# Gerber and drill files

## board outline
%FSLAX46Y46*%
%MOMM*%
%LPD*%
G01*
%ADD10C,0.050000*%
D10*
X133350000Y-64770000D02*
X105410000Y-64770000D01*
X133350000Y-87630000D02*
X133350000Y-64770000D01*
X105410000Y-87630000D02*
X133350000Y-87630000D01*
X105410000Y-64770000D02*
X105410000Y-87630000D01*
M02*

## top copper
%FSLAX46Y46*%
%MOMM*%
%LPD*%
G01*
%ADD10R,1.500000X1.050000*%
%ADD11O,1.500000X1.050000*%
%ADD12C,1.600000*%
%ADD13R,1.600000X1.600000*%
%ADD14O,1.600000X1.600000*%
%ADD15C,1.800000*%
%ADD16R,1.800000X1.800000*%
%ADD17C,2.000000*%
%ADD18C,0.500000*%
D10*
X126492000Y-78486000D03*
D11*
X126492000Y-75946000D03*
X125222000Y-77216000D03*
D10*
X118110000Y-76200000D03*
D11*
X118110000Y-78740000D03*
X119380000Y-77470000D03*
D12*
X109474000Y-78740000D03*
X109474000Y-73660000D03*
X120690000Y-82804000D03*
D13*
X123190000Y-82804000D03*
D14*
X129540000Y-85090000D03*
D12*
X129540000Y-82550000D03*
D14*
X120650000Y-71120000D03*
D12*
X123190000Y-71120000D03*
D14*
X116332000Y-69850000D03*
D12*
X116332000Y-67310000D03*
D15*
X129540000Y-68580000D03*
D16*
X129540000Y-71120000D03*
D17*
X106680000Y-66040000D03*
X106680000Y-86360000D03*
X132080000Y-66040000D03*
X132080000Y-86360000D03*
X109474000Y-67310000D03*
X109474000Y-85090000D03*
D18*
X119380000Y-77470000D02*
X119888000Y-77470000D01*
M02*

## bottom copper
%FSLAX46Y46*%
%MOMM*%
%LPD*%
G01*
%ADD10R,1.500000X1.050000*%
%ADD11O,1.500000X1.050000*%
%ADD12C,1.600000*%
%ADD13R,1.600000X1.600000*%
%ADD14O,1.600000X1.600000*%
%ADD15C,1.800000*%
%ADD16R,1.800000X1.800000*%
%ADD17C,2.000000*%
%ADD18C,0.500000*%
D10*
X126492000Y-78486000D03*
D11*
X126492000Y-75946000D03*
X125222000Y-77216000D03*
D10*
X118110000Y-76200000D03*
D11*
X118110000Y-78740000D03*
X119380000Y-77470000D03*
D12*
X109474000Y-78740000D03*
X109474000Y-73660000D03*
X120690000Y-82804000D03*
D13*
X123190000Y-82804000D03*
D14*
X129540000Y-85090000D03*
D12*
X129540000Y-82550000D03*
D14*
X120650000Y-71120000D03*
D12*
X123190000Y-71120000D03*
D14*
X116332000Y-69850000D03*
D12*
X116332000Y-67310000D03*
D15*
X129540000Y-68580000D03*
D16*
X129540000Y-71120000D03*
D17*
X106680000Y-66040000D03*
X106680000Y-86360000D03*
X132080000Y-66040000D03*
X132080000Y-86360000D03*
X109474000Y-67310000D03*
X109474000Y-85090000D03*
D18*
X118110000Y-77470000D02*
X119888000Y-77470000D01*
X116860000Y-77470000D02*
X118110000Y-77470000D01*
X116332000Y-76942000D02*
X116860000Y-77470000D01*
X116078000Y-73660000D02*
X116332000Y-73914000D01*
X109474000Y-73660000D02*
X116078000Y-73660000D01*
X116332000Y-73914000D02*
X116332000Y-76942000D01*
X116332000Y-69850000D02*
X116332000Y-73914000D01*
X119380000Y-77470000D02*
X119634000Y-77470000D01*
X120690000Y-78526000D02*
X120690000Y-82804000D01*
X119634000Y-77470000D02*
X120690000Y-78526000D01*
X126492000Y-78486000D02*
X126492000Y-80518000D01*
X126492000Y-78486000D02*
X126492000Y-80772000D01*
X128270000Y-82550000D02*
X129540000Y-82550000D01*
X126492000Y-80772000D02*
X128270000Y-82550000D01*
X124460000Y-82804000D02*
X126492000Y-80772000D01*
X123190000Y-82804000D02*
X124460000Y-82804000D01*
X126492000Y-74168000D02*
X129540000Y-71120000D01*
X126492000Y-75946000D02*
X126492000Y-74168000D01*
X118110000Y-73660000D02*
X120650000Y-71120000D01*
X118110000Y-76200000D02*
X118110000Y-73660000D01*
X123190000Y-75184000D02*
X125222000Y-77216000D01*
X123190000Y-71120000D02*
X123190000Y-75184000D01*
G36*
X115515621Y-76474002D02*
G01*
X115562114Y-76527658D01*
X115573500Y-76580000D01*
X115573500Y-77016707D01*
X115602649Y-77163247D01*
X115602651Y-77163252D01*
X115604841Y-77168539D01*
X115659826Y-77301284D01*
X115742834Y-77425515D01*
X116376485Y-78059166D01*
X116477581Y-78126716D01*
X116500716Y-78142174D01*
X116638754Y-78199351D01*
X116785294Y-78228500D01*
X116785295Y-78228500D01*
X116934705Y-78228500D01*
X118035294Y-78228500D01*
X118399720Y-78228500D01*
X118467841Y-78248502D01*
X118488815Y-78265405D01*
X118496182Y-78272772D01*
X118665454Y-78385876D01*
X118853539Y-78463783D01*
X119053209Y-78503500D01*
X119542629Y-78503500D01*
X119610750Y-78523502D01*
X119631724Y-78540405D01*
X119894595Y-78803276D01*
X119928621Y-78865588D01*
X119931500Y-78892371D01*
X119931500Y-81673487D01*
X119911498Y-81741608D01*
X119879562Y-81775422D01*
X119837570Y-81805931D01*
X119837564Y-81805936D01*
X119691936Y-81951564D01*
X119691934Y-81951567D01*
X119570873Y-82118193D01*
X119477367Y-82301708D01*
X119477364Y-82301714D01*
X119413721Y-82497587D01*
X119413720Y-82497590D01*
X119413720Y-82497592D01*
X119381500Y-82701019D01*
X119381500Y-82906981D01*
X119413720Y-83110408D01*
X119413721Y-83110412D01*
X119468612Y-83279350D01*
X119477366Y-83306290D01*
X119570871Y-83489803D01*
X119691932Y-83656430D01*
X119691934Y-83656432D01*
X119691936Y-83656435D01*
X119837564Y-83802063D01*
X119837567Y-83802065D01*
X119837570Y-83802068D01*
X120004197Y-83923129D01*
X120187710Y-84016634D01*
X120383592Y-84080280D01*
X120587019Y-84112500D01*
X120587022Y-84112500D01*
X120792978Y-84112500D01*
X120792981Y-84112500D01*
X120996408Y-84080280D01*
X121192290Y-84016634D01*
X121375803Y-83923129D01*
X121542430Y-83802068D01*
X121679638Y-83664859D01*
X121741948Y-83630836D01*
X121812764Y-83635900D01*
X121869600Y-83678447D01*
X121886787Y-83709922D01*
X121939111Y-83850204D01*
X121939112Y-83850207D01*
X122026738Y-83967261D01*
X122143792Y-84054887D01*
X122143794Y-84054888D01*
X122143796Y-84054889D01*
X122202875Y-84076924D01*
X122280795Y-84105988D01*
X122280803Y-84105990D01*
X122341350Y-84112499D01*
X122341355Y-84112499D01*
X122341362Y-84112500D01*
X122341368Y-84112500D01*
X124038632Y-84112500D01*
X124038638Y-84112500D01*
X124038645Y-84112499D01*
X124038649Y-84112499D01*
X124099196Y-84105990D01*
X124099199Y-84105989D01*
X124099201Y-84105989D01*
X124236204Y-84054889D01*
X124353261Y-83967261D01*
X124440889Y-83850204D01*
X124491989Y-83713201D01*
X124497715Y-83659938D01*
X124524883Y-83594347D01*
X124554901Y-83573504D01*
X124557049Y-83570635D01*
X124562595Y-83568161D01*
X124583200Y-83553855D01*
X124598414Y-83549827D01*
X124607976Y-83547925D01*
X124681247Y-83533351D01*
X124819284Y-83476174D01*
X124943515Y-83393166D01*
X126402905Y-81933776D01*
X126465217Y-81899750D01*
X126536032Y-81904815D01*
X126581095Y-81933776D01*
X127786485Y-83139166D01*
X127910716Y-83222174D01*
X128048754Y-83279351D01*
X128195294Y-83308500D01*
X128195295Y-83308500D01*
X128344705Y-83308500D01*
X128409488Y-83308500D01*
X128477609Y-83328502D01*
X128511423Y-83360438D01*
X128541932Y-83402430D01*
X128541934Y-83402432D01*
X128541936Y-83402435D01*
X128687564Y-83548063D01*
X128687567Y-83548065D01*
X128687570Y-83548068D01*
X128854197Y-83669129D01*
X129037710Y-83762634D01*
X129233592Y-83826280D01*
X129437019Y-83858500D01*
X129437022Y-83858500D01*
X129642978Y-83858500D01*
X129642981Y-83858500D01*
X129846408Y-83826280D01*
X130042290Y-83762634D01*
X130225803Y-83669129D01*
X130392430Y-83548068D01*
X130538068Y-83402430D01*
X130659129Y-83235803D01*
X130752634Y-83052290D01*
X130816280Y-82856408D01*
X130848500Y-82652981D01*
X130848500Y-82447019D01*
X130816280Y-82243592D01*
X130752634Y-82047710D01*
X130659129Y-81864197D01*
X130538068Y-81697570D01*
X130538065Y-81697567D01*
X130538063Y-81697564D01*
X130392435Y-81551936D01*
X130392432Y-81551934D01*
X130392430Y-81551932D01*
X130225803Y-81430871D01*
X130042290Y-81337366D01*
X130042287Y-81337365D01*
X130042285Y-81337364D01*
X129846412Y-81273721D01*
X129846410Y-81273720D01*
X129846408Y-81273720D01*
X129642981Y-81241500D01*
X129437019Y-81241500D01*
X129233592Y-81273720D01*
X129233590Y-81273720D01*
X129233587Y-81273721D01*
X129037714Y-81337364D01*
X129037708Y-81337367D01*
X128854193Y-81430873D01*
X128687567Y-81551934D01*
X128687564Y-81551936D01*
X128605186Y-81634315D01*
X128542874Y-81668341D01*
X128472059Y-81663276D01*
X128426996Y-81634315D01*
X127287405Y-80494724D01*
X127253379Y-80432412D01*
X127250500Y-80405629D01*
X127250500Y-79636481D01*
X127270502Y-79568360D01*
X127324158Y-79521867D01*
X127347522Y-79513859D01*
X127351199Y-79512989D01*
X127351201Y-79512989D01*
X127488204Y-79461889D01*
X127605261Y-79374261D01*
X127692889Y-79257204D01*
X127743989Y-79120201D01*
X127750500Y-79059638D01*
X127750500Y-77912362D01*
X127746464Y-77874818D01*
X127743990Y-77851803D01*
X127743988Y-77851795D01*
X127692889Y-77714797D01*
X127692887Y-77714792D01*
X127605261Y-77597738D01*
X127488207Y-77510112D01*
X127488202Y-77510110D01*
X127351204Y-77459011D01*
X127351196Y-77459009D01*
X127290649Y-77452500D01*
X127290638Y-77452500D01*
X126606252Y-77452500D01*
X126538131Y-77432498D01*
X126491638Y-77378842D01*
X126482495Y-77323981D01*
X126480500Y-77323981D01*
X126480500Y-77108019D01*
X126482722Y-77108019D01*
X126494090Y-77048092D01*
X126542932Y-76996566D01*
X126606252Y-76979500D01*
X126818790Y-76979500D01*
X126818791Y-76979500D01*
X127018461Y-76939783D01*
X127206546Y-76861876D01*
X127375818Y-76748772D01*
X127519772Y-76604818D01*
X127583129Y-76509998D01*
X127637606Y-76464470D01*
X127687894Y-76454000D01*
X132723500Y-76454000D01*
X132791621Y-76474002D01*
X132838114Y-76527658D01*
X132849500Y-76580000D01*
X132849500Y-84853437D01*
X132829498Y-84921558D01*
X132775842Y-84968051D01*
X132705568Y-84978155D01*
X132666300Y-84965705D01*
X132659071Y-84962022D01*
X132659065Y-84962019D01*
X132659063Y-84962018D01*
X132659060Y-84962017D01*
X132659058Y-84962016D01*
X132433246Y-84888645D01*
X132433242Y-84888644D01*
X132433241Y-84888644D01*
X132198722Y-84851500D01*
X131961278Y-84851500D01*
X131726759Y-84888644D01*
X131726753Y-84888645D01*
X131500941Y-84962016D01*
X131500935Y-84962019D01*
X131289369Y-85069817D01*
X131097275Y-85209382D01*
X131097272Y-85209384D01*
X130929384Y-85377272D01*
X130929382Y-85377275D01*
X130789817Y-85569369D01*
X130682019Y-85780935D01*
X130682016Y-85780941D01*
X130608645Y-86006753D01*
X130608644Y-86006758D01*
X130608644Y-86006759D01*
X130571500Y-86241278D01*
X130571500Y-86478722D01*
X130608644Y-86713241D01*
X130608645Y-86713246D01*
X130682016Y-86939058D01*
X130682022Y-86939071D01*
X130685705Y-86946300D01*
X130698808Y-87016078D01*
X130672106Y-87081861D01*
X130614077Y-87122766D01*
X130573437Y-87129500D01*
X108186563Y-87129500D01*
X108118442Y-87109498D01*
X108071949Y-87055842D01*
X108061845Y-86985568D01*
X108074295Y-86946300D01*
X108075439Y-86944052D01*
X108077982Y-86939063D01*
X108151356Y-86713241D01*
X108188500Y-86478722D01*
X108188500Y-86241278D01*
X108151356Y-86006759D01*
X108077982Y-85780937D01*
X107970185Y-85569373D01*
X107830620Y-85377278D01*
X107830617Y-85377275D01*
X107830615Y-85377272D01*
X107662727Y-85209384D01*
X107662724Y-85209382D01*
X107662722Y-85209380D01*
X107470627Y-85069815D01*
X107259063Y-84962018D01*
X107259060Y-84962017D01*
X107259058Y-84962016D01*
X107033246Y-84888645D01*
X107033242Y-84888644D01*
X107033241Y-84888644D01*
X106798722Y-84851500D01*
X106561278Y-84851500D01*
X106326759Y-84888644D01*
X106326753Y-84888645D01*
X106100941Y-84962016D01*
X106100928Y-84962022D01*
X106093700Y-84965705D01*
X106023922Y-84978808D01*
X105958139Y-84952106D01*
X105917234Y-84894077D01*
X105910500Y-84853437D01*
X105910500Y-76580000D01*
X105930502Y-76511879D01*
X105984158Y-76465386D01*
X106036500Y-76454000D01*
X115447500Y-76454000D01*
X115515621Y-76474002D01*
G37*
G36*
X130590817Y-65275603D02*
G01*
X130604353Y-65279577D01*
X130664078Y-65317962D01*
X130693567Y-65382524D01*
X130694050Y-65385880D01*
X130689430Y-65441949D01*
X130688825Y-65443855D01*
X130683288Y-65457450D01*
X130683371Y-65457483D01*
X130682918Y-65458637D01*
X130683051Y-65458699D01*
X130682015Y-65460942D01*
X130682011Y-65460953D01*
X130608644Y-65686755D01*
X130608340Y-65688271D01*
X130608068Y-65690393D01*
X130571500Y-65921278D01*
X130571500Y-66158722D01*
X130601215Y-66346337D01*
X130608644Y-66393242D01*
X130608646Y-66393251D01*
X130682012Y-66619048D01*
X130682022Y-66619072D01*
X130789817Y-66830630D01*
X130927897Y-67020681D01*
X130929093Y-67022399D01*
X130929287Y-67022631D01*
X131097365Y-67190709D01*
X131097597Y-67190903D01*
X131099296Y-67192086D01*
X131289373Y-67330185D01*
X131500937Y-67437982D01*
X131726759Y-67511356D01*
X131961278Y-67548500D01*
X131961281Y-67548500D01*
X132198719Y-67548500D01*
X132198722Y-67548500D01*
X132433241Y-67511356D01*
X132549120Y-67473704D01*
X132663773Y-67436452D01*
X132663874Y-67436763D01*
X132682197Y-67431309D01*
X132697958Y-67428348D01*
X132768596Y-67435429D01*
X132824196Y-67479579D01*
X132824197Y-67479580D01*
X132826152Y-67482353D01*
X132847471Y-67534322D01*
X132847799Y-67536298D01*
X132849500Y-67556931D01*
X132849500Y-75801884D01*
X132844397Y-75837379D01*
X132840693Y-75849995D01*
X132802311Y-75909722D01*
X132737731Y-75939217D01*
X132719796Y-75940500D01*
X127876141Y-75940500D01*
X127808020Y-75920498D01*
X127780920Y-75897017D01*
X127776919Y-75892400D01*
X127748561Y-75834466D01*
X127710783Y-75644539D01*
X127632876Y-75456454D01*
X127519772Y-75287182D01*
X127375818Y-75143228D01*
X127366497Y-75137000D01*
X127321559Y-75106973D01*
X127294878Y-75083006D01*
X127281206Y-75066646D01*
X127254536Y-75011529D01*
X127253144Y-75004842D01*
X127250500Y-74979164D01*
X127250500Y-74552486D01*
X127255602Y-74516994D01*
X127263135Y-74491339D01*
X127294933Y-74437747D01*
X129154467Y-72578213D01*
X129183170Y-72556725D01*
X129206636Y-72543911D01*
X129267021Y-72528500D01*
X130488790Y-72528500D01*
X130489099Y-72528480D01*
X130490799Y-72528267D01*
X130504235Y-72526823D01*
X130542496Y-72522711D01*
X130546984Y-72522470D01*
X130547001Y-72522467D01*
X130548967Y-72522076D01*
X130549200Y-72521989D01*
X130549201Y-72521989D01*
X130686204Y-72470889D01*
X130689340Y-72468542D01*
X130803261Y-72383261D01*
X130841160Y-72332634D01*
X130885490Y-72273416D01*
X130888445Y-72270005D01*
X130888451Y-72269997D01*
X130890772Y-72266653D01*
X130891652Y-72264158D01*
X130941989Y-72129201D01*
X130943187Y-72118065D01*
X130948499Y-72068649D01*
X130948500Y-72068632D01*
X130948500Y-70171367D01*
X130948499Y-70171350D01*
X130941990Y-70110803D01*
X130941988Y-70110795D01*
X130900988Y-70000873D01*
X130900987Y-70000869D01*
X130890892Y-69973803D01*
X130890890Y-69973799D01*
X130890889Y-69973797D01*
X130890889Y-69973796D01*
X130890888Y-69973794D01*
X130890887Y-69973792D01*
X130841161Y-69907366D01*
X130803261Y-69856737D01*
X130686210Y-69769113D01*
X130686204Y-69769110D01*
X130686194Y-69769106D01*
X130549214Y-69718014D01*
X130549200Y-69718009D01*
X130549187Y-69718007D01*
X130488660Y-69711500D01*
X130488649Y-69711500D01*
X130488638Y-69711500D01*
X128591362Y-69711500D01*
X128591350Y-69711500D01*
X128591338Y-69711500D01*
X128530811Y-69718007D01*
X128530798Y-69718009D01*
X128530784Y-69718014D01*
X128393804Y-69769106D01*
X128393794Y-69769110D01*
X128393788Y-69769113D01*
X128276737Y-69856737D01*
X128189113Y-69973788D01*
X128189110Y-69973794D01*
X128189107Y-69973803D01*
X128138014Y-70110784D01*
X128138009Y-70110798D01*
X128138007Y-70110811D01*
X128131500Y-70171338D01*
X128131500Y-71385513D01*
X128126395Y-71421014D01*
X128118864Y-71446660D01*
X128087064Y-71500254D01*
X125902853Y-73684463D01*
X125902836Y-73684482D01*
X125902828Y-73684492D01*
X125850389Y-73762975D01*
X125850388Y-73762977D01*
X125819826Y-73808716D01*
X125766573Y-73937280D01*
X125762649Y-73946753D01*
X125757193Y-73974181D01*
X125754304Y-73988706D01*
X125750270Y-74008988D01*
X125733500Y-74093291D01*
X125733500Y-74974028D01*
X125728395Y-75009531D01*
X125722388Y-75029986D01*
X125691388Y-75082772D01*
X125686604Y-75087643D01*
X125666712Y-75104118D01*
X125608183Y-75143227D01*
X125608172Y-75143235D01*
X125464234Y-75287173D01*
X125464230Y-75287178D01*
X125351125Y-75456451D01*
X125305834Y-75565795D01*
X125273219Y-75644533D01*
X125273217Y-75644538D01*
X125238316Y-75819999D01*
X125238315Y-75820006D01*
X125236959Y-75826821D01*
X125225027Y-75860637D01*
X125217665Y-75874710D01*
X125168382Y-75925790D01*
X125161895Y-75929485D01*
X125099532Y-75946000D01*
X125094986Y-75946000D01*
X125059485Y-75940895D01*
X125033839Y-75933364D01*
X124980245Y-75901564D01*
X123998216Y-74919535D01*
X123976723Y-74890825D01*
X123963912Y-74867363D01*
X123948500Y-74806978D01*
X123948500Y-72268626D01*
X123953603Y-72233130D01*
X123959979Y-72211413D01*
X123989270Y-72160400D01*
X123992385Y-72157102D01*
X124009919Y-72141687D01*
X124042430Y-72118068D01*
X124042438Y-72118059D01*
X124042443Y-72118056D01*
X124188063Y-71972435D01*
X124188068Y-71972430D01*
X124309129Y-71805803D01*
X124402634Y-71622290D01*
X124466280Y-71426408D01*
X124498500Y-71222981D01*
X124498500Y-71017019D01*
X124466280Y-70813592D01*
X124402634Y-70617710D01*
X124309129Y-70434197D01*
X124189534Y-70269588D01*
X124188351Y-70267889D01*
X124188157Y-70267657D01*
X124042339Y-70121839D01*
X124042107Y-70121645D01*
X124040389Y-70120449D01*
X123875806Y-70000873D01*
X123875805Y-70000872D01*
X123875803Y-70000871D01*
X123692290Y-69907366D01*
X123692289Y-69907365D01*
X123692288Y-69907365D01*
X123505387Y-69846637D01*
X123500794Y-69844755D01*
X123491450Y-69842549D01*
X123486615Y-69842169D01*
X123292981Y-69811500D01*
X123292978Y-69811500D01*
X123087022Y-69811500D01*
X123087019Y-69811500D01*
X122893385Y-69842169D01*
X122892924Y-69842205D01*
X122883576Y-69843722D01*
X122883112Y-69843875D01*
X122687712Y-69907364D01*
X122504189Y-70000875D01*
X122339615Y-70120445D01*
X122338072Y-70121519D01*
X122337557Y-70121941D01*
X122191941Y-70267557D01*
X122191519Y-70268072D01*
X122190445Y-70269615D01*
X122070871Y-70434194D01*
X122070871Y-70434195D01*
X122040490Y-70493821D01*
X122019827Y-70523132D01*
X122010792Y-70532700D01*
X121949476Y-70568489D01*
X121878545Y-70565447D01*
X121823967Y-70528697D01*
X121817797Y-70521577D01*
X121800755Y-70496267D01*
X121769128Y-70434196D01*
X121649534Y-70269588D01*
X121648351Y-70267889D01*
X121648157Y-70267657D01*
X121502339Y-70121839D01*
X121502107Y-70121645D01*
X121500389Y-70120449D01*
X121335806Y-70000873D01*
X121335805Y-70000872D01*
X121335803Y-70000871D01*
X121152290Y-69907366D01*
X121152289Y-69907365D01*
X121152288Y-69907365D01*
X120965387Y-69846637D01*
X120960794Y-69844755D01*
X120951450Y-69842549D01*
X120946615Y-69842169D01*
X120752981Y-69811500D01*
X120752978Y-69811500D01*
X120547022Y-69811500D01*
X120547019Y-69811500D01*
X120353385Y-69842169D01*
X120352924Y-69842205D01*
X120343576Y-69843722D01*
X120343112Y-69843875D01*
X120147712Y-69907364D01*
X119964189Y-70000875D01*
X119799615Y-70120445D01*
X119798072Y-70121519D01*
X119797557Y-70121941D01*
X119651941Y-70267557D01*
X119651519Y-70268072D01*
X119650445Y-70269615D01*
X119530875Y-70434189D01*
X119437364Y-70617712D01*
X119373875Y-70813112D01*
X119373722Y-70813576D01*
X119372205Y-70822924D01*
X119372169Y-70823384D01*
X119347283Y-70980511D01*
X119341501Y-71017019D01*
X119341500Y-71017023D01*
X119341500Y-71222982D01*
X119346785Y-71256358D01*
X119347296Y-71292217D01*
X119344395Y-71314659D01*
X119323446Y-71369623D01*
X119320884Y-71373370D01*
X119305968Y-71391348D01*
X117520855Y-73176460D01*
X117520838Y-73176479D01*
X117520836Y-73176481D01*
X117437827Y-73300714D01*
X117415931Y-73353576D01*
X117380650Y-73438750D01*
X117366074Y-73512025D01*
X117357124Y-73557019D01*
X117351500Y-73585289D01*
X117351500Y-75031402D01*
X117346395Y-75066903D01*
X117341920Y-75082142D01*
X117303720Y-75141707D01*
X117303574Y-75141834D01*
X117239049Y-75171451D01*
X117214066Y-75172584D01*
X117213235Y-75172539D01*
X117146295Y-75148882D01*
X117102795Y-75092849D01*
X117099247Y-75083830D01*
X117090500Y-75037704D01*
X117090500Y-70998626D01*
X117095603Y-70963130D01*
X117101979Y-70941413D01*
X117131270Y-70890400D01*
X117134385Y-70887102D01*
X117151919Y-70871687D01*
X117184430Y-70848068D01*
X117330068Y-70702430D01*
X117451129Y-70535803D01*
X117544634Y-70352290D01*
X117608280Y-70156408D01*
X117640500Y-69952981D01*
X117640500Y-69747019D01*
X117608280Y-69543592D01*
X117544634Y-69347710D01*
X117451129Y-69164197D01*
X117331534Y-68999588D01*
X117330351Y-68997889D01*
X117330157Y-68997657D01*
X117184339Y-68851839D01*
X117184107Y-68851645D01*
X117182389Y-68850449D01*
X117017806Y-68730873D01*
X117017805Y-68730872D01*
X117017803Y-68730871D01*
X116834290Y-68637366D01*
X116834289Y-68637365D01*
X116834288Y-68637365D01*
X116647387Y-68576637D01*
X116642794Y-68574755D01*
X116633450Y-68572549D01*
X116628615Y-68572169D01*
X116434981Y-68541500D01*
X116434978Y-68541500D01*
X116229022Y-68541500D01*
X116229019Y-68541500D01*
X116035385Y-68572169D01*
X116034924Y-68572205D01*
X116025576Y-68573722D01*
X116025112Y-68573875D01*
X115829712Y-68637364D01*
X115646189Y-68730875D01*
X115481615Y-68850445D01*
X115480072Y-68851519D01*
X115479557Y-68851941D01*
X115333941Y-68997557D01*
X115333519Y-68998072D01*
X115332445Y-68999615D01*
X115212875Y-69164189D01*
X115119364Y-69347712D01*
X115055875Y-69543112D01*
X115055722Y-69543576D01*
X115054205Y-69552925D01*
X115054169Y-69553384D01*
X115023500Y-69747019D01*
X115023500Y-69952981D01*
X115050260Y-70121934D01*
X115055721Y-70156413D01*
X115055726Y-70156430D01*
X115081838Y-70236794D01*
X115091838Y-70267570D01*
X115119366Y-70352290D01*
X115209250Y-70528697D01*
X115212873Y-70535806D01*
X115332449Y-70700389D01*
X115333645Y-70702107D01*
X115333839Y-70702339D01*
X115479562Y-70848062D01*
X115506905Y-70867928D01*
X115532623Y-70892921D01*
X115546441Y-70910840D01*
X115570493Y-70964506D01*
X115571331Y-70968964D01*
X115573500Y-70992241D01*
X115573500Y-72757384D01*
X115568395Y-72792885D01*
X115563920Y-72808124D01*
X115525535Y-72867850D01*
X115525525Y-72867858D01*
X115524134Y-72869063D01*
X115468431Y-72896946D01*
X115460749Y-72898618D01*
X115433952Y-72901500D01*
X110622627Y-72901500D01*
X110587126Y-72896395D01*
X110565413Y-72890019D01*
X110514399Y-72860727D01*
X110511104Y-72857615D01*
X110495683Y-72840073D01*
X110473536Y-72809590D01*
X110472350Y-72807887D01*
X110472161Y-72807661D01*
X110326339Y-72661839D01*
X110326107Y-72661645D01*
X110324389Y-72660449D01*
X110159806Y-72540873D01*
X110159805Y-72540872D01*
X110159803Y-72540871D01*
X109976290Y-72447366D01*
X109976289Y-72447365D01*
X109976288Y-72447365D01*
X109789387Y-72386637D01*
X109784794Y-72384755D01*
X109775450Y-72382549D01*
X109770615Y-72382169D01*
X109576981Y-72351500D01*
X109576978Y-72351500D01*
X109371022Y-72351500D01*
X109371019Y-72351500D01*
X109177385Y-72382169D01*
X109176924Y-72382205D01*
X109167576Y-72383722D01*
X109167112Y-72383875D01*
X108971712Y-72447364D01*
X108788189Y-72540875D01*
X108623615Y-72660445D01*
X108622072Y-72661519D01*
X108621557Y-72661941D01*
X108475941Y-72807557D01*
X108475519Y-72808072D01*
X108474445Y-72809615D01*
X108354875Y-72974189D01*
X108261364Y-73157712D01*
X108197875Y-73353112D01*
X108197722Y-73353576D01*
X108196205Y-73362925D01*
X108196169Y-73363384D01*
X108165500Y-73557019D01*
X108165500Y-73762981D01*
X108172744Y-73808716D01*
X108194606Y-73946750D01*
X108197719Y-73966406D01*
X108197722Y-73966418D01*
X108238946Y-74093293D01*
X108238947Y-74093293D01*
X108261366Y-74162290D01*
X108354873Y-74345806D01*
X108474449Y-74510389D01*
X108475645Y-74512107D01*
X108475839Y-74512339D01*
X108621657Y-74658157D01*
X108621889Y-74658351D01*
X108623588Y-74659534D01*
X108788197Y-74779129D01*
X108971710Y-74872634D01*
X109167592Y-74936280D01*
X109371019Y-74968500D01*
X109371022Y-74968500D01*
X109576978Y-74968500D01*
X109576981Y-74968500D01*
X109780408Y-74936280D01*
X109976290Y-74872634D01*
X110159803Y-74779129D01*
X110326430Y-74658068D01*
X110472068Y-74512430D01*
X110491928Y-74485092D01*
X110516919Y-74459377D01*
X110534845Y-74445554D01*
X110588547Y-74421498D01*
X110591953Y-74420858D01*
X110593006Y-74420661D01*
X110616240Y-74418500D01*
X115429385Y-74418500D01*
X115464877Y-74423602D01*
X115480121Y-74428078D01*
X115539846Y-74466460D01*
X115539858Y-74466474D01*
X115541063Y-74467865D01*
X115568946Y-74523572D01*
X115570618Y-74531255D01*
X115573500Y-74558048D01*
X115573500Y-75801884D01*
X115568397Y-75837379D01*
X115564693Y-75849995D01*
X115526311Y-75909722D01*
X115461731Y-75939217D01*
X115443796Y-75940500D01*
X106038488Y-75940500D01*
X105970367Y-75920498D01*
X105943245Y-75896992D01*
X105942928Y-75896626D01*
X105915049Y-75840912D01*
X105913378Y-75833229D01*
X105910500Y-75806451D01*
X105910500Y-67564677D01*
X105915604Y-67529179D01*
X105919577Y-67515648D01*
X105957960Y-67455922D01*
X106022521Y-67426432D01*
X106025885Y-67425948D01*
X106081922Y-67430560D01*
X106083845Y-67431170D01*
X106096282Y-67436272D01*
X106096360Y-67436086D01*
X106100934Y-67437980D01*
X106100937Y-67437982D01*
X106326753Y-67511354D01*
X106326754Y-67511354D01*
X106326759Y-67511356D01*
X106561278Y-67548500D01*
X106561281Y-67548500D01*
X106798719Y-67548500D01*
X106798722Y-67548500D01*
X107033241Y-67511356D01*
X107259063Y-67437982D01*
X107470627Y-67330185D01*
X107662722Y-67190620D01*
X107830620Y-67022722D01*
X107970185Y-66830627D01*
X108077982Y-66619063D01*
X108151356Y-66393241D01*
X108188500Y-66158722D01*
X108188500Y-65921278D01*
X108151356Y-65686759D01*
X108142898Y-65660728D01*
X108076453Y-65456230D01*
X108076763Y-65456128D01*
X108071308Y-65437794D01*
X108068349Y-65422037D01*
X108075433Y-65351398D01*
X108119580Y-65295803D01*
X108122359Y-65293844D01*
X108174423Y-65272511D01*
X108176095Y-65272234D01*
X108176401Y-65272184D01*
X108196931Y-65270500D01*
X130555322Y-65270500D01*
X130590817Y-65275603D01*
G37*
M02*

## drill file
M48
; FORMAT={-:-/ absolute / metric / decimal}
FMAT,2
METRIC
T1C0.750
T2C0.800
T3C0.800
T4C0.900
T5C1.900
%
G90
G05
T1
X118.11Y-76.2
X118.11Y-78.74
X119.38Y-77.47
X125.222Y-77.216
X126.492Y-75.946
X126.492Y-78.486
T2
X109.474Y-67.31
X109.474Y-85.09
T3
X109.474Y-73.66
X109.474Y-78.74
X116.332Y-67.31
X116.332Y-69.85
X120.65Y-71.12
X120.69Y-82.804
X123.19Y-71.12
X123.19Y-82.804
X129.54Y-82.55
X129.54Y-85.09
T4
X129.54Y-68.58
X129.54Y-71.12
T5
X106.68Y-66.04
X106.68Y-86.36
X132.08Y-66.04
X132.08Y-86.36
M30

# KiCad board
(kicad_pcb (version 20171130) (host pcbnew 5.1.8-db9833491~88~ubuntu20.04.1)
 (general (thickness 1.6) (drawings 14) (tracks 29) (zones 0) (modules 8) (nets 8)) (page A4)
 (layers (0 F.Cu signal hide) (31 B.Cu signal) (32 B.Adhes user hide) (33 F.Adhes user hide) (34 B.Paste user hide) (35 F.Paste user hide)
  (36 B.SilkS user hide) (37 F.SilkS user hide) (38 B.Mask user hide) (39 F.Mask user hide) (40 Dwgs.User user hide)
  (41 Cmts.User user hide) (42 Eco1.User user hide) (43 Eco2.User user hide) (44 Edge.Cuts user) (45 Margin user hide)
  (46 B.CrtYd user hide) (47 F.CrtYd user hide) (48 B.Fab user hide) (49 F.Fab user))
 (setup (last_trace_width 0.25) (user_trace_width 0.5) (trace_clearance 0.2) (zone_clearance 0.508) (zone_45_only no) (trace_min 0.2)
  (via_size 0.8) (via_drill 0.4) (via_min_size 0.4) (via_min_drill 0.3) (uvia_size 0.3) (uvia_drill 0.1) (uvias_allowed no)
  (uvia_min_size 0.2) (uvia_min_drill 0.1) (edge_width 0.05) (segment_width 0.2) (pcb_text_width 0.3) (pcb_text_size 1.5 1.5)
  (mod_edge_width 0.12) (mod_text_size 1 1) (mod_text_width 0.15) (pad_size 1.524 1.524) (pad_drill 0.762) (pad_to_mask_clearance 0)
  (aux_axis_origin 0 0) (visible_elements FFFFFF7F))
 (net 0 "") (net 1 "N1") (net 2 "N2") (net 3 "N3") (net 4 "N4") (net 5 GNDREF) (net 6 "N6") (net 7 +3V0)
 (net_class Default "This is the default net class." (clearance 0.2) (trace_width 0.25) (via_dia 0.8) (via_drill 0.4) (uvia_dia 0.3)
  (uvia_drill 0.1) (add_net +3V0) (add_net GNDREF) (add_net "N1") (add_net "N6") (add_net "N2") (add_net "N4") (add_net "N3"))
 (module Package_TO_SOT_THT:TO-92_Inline (layer F.Cu) (at 126.492 78.486 90)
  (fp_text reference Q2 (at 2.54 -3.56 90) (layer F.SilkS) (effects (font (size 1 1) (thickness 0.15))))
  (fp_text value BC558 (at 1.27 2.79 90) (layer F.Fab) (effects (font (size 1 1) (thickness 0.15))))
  (pad 1 thru_hole rect (at 0 0 90) (size 1.05 1.5) (drill 0.75) (layers *.Cu *.Mask) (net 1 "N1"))
  (pad 3 thru_hole oval (at 2.54 0 90) (size 1.05 1.5) (drill 0.75) (layers *.Cu *.Mask) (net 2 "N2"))
  (pad 2 thru_hole oval (at 1.27 -1.27 90) (size 1.05 1.5) (drill 0.75) (layers *.Cu *.Mask) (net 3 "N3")))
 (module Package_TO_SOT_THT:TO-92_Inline (layer F.Cu) (at 118.11 76.2 270)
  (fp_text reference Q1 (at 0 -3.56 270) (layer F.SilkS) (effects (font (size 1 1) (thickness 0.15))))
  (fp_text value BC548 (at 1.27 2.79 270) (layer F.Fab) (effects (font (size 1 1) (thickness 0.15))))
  (pad 1 thru_hole rect (at 0 0 270) (size 1.05 1.5) (drill 0.75) (layers *.Cu *.Mask) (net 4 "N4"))
  (pad 3 thru_hole oval (at 2.54 0 270) (size 1.05 1.5) (drill 0.75) (layers *.Cu *.Mask) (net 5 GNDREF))
  (pad 2 thru_hole oval (at 1.27 -1.27 270) (size 1.05 1.5) (drill 0.75) (layers *.Cu *.Mask) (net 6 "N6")))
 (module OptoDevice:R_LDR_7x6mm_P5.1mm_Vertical (layer F.Cu) (at 109.474 73.66 270)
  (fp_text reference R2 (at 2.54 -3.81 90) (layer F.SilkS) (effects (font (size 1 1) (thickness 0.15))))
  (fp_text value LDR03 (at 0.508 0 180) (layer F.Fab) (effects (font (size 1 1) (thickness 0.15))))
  (pad 2 thru_hole circle (at 5.08 0 270) (size 1.6 1.6) (drill 0.8) (layers *.Cu *.Mask) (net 5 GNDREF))
  (pad 1 thru_hole circle (at 0 0 270) (size 1.6 1.6) (drill 0.8) (layers *.Cu *.Mask) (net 6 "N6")))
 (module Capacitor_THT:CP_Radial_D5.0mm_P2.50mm (layer F.Cu) (at 123.19 82.804 180)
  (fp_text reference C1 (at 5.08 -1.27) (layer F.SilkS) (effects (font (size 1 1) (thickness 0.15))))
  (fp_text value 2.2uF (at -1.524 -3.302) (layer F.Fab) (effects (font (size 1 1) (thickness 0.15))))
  (pad 2 thru_hole circle (at 2.5 0 180) (size 1.6 1.6) (drill 0.8) (layers *.Cu *.Mask) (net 6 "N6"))
  (pad 1 thru_hole rect (at 0 0 180) (size 1.6 1.6) (drill 0.8) (layers *.Cu *.Mask) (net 1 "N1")))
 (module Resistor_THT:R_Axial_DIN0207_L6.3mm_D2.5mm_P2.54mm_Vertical (layer F.Cu) (at 129.54 82.55 270)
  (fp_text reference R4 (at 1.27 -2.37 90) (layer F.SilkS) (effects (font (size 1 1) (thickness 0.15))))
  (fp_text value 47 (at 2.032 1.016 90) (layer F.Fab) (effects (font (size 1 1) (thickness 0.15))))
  (pad 2 thru_hole oval (at 2.54 0 270) (size 1.6 1.6) (drill 0.8) (layers *.Cu *.Mask) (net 5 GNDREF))
  (pad 1 thru_hole circle (at 0 0 270) (size 1.6 1.6) (drill 0.8) (layers *.Cu *.Mask) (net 1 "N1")))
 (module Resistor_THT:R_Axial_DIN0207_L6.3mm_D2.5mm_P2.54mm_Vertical (layer F.Cu) (at 123.19 71.12 180)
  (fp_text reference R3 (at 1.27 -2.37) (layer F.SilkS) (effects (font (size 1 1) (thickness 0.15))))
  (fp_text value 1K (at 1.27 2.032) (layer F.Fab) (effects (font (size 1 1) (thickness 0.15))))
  (pad 2 thru_hole oval (at 2.54 0 180) (size 1.6 1.6) (drill 0.8) (layers *.Cu *.Mask) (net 4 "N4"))
  (pad 1 thru_hole circle (at 0 0 180) (size 1.6 1.6) (drill 0.8) (layers *.Cu *.Mask) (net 3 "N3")))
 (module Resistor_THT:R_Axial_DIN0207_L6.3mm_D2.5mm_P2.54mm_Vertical (layer F.Cu) (at 116.332 67.31 270)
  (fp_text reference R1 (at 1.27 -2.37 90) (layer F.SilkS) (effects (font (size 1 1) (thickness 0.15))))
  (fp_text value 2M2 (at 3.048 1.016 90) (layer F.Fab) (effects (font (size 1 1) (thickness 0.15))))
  (pad 2 thru_hole oval (at 2.54 0 270) (size 1.6 1.6) (drill 0.8) (layers *.Cu *.Mask) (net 6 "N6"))
  (pad 1 thru_hole circle (at 0 0 270) (size 1.6 1.6) (drill 0.8) (layers *.Cu *.Mask) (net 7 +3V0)))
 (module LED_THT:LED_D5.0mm (layer F.Cu) (at 129.54 71.12 90)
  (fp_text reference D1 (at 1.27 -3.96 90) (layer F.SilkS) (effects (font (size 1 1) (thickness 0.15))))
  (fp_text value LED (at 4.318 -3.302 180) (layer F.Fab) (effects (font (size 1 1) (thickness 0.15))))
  (pad 2 thru_hole circle (at 2.54 0 90) (size 1.8 1.8) (drill 0.9) (layers *.Cu *.Mask) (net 7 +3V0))
  (pad 1 thru_hole rect (at 0 0 90) (size 1.8 1.8) (drill 0.9) (layers *.Cu *.Mask) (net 2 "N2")))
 (gr_line (start 133.35 64.77) (end 105.41 64.77) (layer Edge.Cuts) (width 0.05))
 (gr_line (start 133.35 87.63) (end 133.35 64.77) (layer Edge.Cuts) (width 0.05))
 (gr_line (start 105.41 87.63) (end 133.35 87.63) (layer Edge.Cuts) (width 0.05))
 (gr_line (start 105.41 64.77) (end 105.41 87.63) (layer Edge.Cuts) (width 0.05))
 (via (at 106.68 66.04) (size 2) (drill 1.9) (layers F.Cu B.Cu) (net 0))
 (via (at 106.68 86.36) (size 2) (drill 1.9) (layers F.Cu B.Cu) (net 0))
 (via (at 132.08 66.04) (size 2) (drill 1.9) (layers F.Cu B.Cu) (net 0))
 (via (at 132.08 86.36) (size 2) (drill 1.9) (layers F.Cu B.Cu) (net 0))
 (segment (start 118.11 77.47) (end 119.888 77.47) (width 0.5) (layer B.Cu) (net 6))
 (segment (start 116.86 77.47) (end 118.11 77.47) (width 0.5) (layer B.Cu) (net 6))
 (segment (start 116.332 76.942) (end 116.86 77.47) (width 0.5) (layer B.Cu) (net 6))
 (segment (start 116.078 73.66) (end 116.332 73.914) (width 0.5) (layer B.Cu) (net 6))
 (segment (start 109.474 73.66) (end 116.078 73.66) (width 0.5) (layer B.Cu) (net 6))
 (segment (start 116.332 73.914) (end 116.332 76.942) (width 0.5) (layer B.Cu) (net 6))
 (segment (start 116.332 69.85) (end 116.332 73.914) (width 0.5) (layer B.Cu) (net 6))
 (segment (start 119.38 77.47) (end 119.888 77.47) (width 0.5) (layer F.Cu) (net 6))
 (segment (start 119.38 77.47) (end 119.634 77.47) (width 0.5) (layer B.Cu) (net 6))
 (segment (start 120.69 78.526) (end 120.69 82.804) (width 0.5) (layer B.Cu) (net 6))
 (segment (start 119.634 77.47) (end 120.69 78.526) (width 0.5) (layer B.Cu) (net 6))
 (segment (start 126.492 78.486) (end 126.492 80.518) (width 0.5) (layer B.Cu) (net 1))
 (segment (start 126.492 78.486) (end 126.492 80.772) (width 0.5) (layer B.Cu) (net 1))
 (segment (start 128.27 82.55) (end 129.54 82.55) (width 0.5) (layer B.Cu) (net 1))
 (segment (start 126.492 80.772) (end 128.27 82.55) (width 0.5) (layer B.Cu) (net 1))
 (segment (start 124.46 82.804) (end 126.492 80.772) (width 0.5) (layer B.Cu) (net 1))
 (segment (start 123.19 82.804) (end 124.46 82.804) (width 0.5) (layer B.Cu) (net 1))
 (segment (start 126.492 74.168) (end 129.54 71.12) (width 0.5) (layer B.Cu) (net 2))
 (segment (start 126.492 75.946) (end 126.492 74.168) (width 0.5) (layer B.Cu) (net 2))
 (segment (start 118.11 73.66) (end 120.65 71.12) (width 0.5) (layer B.Cu) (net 4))
 (segment (start 118.11 76.2) (end 118.11 73.66) (width 0.5) (layer B.Cu) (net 4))
 (segment (start 123.19 75.184) (end 125.222 77.216) (width 0.5) (layer B.Cu) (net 3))
 (segment (start 123.19 71.12) (end 123.19 75.184) (width 0.5) (layer B.Cu) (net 3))
 (via (at 109.474 67.31) (size 2) (drill 0.8) (layers F.Cu B.Cu) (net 7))
 (via (at 109.474 85.09) (size 2) (drill 0.8) (layers F.Cu B.Cu) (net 5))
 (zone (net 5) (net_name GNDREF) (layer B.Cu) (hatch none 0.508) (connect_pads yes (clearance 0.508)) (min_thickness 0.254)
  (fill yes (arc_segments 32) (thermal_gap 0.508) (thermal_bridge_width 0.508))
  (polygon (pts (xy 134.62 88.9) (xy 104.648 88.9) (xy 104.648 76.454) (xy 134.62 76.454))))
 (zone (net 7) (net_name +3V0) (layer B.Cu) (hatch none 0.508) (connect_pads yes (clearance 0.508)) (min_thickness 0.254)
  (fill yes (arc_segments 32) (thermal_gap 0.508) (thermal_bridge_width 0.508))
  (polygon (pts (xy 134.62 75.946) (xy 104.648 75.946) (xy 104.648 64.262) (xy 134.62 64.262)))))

